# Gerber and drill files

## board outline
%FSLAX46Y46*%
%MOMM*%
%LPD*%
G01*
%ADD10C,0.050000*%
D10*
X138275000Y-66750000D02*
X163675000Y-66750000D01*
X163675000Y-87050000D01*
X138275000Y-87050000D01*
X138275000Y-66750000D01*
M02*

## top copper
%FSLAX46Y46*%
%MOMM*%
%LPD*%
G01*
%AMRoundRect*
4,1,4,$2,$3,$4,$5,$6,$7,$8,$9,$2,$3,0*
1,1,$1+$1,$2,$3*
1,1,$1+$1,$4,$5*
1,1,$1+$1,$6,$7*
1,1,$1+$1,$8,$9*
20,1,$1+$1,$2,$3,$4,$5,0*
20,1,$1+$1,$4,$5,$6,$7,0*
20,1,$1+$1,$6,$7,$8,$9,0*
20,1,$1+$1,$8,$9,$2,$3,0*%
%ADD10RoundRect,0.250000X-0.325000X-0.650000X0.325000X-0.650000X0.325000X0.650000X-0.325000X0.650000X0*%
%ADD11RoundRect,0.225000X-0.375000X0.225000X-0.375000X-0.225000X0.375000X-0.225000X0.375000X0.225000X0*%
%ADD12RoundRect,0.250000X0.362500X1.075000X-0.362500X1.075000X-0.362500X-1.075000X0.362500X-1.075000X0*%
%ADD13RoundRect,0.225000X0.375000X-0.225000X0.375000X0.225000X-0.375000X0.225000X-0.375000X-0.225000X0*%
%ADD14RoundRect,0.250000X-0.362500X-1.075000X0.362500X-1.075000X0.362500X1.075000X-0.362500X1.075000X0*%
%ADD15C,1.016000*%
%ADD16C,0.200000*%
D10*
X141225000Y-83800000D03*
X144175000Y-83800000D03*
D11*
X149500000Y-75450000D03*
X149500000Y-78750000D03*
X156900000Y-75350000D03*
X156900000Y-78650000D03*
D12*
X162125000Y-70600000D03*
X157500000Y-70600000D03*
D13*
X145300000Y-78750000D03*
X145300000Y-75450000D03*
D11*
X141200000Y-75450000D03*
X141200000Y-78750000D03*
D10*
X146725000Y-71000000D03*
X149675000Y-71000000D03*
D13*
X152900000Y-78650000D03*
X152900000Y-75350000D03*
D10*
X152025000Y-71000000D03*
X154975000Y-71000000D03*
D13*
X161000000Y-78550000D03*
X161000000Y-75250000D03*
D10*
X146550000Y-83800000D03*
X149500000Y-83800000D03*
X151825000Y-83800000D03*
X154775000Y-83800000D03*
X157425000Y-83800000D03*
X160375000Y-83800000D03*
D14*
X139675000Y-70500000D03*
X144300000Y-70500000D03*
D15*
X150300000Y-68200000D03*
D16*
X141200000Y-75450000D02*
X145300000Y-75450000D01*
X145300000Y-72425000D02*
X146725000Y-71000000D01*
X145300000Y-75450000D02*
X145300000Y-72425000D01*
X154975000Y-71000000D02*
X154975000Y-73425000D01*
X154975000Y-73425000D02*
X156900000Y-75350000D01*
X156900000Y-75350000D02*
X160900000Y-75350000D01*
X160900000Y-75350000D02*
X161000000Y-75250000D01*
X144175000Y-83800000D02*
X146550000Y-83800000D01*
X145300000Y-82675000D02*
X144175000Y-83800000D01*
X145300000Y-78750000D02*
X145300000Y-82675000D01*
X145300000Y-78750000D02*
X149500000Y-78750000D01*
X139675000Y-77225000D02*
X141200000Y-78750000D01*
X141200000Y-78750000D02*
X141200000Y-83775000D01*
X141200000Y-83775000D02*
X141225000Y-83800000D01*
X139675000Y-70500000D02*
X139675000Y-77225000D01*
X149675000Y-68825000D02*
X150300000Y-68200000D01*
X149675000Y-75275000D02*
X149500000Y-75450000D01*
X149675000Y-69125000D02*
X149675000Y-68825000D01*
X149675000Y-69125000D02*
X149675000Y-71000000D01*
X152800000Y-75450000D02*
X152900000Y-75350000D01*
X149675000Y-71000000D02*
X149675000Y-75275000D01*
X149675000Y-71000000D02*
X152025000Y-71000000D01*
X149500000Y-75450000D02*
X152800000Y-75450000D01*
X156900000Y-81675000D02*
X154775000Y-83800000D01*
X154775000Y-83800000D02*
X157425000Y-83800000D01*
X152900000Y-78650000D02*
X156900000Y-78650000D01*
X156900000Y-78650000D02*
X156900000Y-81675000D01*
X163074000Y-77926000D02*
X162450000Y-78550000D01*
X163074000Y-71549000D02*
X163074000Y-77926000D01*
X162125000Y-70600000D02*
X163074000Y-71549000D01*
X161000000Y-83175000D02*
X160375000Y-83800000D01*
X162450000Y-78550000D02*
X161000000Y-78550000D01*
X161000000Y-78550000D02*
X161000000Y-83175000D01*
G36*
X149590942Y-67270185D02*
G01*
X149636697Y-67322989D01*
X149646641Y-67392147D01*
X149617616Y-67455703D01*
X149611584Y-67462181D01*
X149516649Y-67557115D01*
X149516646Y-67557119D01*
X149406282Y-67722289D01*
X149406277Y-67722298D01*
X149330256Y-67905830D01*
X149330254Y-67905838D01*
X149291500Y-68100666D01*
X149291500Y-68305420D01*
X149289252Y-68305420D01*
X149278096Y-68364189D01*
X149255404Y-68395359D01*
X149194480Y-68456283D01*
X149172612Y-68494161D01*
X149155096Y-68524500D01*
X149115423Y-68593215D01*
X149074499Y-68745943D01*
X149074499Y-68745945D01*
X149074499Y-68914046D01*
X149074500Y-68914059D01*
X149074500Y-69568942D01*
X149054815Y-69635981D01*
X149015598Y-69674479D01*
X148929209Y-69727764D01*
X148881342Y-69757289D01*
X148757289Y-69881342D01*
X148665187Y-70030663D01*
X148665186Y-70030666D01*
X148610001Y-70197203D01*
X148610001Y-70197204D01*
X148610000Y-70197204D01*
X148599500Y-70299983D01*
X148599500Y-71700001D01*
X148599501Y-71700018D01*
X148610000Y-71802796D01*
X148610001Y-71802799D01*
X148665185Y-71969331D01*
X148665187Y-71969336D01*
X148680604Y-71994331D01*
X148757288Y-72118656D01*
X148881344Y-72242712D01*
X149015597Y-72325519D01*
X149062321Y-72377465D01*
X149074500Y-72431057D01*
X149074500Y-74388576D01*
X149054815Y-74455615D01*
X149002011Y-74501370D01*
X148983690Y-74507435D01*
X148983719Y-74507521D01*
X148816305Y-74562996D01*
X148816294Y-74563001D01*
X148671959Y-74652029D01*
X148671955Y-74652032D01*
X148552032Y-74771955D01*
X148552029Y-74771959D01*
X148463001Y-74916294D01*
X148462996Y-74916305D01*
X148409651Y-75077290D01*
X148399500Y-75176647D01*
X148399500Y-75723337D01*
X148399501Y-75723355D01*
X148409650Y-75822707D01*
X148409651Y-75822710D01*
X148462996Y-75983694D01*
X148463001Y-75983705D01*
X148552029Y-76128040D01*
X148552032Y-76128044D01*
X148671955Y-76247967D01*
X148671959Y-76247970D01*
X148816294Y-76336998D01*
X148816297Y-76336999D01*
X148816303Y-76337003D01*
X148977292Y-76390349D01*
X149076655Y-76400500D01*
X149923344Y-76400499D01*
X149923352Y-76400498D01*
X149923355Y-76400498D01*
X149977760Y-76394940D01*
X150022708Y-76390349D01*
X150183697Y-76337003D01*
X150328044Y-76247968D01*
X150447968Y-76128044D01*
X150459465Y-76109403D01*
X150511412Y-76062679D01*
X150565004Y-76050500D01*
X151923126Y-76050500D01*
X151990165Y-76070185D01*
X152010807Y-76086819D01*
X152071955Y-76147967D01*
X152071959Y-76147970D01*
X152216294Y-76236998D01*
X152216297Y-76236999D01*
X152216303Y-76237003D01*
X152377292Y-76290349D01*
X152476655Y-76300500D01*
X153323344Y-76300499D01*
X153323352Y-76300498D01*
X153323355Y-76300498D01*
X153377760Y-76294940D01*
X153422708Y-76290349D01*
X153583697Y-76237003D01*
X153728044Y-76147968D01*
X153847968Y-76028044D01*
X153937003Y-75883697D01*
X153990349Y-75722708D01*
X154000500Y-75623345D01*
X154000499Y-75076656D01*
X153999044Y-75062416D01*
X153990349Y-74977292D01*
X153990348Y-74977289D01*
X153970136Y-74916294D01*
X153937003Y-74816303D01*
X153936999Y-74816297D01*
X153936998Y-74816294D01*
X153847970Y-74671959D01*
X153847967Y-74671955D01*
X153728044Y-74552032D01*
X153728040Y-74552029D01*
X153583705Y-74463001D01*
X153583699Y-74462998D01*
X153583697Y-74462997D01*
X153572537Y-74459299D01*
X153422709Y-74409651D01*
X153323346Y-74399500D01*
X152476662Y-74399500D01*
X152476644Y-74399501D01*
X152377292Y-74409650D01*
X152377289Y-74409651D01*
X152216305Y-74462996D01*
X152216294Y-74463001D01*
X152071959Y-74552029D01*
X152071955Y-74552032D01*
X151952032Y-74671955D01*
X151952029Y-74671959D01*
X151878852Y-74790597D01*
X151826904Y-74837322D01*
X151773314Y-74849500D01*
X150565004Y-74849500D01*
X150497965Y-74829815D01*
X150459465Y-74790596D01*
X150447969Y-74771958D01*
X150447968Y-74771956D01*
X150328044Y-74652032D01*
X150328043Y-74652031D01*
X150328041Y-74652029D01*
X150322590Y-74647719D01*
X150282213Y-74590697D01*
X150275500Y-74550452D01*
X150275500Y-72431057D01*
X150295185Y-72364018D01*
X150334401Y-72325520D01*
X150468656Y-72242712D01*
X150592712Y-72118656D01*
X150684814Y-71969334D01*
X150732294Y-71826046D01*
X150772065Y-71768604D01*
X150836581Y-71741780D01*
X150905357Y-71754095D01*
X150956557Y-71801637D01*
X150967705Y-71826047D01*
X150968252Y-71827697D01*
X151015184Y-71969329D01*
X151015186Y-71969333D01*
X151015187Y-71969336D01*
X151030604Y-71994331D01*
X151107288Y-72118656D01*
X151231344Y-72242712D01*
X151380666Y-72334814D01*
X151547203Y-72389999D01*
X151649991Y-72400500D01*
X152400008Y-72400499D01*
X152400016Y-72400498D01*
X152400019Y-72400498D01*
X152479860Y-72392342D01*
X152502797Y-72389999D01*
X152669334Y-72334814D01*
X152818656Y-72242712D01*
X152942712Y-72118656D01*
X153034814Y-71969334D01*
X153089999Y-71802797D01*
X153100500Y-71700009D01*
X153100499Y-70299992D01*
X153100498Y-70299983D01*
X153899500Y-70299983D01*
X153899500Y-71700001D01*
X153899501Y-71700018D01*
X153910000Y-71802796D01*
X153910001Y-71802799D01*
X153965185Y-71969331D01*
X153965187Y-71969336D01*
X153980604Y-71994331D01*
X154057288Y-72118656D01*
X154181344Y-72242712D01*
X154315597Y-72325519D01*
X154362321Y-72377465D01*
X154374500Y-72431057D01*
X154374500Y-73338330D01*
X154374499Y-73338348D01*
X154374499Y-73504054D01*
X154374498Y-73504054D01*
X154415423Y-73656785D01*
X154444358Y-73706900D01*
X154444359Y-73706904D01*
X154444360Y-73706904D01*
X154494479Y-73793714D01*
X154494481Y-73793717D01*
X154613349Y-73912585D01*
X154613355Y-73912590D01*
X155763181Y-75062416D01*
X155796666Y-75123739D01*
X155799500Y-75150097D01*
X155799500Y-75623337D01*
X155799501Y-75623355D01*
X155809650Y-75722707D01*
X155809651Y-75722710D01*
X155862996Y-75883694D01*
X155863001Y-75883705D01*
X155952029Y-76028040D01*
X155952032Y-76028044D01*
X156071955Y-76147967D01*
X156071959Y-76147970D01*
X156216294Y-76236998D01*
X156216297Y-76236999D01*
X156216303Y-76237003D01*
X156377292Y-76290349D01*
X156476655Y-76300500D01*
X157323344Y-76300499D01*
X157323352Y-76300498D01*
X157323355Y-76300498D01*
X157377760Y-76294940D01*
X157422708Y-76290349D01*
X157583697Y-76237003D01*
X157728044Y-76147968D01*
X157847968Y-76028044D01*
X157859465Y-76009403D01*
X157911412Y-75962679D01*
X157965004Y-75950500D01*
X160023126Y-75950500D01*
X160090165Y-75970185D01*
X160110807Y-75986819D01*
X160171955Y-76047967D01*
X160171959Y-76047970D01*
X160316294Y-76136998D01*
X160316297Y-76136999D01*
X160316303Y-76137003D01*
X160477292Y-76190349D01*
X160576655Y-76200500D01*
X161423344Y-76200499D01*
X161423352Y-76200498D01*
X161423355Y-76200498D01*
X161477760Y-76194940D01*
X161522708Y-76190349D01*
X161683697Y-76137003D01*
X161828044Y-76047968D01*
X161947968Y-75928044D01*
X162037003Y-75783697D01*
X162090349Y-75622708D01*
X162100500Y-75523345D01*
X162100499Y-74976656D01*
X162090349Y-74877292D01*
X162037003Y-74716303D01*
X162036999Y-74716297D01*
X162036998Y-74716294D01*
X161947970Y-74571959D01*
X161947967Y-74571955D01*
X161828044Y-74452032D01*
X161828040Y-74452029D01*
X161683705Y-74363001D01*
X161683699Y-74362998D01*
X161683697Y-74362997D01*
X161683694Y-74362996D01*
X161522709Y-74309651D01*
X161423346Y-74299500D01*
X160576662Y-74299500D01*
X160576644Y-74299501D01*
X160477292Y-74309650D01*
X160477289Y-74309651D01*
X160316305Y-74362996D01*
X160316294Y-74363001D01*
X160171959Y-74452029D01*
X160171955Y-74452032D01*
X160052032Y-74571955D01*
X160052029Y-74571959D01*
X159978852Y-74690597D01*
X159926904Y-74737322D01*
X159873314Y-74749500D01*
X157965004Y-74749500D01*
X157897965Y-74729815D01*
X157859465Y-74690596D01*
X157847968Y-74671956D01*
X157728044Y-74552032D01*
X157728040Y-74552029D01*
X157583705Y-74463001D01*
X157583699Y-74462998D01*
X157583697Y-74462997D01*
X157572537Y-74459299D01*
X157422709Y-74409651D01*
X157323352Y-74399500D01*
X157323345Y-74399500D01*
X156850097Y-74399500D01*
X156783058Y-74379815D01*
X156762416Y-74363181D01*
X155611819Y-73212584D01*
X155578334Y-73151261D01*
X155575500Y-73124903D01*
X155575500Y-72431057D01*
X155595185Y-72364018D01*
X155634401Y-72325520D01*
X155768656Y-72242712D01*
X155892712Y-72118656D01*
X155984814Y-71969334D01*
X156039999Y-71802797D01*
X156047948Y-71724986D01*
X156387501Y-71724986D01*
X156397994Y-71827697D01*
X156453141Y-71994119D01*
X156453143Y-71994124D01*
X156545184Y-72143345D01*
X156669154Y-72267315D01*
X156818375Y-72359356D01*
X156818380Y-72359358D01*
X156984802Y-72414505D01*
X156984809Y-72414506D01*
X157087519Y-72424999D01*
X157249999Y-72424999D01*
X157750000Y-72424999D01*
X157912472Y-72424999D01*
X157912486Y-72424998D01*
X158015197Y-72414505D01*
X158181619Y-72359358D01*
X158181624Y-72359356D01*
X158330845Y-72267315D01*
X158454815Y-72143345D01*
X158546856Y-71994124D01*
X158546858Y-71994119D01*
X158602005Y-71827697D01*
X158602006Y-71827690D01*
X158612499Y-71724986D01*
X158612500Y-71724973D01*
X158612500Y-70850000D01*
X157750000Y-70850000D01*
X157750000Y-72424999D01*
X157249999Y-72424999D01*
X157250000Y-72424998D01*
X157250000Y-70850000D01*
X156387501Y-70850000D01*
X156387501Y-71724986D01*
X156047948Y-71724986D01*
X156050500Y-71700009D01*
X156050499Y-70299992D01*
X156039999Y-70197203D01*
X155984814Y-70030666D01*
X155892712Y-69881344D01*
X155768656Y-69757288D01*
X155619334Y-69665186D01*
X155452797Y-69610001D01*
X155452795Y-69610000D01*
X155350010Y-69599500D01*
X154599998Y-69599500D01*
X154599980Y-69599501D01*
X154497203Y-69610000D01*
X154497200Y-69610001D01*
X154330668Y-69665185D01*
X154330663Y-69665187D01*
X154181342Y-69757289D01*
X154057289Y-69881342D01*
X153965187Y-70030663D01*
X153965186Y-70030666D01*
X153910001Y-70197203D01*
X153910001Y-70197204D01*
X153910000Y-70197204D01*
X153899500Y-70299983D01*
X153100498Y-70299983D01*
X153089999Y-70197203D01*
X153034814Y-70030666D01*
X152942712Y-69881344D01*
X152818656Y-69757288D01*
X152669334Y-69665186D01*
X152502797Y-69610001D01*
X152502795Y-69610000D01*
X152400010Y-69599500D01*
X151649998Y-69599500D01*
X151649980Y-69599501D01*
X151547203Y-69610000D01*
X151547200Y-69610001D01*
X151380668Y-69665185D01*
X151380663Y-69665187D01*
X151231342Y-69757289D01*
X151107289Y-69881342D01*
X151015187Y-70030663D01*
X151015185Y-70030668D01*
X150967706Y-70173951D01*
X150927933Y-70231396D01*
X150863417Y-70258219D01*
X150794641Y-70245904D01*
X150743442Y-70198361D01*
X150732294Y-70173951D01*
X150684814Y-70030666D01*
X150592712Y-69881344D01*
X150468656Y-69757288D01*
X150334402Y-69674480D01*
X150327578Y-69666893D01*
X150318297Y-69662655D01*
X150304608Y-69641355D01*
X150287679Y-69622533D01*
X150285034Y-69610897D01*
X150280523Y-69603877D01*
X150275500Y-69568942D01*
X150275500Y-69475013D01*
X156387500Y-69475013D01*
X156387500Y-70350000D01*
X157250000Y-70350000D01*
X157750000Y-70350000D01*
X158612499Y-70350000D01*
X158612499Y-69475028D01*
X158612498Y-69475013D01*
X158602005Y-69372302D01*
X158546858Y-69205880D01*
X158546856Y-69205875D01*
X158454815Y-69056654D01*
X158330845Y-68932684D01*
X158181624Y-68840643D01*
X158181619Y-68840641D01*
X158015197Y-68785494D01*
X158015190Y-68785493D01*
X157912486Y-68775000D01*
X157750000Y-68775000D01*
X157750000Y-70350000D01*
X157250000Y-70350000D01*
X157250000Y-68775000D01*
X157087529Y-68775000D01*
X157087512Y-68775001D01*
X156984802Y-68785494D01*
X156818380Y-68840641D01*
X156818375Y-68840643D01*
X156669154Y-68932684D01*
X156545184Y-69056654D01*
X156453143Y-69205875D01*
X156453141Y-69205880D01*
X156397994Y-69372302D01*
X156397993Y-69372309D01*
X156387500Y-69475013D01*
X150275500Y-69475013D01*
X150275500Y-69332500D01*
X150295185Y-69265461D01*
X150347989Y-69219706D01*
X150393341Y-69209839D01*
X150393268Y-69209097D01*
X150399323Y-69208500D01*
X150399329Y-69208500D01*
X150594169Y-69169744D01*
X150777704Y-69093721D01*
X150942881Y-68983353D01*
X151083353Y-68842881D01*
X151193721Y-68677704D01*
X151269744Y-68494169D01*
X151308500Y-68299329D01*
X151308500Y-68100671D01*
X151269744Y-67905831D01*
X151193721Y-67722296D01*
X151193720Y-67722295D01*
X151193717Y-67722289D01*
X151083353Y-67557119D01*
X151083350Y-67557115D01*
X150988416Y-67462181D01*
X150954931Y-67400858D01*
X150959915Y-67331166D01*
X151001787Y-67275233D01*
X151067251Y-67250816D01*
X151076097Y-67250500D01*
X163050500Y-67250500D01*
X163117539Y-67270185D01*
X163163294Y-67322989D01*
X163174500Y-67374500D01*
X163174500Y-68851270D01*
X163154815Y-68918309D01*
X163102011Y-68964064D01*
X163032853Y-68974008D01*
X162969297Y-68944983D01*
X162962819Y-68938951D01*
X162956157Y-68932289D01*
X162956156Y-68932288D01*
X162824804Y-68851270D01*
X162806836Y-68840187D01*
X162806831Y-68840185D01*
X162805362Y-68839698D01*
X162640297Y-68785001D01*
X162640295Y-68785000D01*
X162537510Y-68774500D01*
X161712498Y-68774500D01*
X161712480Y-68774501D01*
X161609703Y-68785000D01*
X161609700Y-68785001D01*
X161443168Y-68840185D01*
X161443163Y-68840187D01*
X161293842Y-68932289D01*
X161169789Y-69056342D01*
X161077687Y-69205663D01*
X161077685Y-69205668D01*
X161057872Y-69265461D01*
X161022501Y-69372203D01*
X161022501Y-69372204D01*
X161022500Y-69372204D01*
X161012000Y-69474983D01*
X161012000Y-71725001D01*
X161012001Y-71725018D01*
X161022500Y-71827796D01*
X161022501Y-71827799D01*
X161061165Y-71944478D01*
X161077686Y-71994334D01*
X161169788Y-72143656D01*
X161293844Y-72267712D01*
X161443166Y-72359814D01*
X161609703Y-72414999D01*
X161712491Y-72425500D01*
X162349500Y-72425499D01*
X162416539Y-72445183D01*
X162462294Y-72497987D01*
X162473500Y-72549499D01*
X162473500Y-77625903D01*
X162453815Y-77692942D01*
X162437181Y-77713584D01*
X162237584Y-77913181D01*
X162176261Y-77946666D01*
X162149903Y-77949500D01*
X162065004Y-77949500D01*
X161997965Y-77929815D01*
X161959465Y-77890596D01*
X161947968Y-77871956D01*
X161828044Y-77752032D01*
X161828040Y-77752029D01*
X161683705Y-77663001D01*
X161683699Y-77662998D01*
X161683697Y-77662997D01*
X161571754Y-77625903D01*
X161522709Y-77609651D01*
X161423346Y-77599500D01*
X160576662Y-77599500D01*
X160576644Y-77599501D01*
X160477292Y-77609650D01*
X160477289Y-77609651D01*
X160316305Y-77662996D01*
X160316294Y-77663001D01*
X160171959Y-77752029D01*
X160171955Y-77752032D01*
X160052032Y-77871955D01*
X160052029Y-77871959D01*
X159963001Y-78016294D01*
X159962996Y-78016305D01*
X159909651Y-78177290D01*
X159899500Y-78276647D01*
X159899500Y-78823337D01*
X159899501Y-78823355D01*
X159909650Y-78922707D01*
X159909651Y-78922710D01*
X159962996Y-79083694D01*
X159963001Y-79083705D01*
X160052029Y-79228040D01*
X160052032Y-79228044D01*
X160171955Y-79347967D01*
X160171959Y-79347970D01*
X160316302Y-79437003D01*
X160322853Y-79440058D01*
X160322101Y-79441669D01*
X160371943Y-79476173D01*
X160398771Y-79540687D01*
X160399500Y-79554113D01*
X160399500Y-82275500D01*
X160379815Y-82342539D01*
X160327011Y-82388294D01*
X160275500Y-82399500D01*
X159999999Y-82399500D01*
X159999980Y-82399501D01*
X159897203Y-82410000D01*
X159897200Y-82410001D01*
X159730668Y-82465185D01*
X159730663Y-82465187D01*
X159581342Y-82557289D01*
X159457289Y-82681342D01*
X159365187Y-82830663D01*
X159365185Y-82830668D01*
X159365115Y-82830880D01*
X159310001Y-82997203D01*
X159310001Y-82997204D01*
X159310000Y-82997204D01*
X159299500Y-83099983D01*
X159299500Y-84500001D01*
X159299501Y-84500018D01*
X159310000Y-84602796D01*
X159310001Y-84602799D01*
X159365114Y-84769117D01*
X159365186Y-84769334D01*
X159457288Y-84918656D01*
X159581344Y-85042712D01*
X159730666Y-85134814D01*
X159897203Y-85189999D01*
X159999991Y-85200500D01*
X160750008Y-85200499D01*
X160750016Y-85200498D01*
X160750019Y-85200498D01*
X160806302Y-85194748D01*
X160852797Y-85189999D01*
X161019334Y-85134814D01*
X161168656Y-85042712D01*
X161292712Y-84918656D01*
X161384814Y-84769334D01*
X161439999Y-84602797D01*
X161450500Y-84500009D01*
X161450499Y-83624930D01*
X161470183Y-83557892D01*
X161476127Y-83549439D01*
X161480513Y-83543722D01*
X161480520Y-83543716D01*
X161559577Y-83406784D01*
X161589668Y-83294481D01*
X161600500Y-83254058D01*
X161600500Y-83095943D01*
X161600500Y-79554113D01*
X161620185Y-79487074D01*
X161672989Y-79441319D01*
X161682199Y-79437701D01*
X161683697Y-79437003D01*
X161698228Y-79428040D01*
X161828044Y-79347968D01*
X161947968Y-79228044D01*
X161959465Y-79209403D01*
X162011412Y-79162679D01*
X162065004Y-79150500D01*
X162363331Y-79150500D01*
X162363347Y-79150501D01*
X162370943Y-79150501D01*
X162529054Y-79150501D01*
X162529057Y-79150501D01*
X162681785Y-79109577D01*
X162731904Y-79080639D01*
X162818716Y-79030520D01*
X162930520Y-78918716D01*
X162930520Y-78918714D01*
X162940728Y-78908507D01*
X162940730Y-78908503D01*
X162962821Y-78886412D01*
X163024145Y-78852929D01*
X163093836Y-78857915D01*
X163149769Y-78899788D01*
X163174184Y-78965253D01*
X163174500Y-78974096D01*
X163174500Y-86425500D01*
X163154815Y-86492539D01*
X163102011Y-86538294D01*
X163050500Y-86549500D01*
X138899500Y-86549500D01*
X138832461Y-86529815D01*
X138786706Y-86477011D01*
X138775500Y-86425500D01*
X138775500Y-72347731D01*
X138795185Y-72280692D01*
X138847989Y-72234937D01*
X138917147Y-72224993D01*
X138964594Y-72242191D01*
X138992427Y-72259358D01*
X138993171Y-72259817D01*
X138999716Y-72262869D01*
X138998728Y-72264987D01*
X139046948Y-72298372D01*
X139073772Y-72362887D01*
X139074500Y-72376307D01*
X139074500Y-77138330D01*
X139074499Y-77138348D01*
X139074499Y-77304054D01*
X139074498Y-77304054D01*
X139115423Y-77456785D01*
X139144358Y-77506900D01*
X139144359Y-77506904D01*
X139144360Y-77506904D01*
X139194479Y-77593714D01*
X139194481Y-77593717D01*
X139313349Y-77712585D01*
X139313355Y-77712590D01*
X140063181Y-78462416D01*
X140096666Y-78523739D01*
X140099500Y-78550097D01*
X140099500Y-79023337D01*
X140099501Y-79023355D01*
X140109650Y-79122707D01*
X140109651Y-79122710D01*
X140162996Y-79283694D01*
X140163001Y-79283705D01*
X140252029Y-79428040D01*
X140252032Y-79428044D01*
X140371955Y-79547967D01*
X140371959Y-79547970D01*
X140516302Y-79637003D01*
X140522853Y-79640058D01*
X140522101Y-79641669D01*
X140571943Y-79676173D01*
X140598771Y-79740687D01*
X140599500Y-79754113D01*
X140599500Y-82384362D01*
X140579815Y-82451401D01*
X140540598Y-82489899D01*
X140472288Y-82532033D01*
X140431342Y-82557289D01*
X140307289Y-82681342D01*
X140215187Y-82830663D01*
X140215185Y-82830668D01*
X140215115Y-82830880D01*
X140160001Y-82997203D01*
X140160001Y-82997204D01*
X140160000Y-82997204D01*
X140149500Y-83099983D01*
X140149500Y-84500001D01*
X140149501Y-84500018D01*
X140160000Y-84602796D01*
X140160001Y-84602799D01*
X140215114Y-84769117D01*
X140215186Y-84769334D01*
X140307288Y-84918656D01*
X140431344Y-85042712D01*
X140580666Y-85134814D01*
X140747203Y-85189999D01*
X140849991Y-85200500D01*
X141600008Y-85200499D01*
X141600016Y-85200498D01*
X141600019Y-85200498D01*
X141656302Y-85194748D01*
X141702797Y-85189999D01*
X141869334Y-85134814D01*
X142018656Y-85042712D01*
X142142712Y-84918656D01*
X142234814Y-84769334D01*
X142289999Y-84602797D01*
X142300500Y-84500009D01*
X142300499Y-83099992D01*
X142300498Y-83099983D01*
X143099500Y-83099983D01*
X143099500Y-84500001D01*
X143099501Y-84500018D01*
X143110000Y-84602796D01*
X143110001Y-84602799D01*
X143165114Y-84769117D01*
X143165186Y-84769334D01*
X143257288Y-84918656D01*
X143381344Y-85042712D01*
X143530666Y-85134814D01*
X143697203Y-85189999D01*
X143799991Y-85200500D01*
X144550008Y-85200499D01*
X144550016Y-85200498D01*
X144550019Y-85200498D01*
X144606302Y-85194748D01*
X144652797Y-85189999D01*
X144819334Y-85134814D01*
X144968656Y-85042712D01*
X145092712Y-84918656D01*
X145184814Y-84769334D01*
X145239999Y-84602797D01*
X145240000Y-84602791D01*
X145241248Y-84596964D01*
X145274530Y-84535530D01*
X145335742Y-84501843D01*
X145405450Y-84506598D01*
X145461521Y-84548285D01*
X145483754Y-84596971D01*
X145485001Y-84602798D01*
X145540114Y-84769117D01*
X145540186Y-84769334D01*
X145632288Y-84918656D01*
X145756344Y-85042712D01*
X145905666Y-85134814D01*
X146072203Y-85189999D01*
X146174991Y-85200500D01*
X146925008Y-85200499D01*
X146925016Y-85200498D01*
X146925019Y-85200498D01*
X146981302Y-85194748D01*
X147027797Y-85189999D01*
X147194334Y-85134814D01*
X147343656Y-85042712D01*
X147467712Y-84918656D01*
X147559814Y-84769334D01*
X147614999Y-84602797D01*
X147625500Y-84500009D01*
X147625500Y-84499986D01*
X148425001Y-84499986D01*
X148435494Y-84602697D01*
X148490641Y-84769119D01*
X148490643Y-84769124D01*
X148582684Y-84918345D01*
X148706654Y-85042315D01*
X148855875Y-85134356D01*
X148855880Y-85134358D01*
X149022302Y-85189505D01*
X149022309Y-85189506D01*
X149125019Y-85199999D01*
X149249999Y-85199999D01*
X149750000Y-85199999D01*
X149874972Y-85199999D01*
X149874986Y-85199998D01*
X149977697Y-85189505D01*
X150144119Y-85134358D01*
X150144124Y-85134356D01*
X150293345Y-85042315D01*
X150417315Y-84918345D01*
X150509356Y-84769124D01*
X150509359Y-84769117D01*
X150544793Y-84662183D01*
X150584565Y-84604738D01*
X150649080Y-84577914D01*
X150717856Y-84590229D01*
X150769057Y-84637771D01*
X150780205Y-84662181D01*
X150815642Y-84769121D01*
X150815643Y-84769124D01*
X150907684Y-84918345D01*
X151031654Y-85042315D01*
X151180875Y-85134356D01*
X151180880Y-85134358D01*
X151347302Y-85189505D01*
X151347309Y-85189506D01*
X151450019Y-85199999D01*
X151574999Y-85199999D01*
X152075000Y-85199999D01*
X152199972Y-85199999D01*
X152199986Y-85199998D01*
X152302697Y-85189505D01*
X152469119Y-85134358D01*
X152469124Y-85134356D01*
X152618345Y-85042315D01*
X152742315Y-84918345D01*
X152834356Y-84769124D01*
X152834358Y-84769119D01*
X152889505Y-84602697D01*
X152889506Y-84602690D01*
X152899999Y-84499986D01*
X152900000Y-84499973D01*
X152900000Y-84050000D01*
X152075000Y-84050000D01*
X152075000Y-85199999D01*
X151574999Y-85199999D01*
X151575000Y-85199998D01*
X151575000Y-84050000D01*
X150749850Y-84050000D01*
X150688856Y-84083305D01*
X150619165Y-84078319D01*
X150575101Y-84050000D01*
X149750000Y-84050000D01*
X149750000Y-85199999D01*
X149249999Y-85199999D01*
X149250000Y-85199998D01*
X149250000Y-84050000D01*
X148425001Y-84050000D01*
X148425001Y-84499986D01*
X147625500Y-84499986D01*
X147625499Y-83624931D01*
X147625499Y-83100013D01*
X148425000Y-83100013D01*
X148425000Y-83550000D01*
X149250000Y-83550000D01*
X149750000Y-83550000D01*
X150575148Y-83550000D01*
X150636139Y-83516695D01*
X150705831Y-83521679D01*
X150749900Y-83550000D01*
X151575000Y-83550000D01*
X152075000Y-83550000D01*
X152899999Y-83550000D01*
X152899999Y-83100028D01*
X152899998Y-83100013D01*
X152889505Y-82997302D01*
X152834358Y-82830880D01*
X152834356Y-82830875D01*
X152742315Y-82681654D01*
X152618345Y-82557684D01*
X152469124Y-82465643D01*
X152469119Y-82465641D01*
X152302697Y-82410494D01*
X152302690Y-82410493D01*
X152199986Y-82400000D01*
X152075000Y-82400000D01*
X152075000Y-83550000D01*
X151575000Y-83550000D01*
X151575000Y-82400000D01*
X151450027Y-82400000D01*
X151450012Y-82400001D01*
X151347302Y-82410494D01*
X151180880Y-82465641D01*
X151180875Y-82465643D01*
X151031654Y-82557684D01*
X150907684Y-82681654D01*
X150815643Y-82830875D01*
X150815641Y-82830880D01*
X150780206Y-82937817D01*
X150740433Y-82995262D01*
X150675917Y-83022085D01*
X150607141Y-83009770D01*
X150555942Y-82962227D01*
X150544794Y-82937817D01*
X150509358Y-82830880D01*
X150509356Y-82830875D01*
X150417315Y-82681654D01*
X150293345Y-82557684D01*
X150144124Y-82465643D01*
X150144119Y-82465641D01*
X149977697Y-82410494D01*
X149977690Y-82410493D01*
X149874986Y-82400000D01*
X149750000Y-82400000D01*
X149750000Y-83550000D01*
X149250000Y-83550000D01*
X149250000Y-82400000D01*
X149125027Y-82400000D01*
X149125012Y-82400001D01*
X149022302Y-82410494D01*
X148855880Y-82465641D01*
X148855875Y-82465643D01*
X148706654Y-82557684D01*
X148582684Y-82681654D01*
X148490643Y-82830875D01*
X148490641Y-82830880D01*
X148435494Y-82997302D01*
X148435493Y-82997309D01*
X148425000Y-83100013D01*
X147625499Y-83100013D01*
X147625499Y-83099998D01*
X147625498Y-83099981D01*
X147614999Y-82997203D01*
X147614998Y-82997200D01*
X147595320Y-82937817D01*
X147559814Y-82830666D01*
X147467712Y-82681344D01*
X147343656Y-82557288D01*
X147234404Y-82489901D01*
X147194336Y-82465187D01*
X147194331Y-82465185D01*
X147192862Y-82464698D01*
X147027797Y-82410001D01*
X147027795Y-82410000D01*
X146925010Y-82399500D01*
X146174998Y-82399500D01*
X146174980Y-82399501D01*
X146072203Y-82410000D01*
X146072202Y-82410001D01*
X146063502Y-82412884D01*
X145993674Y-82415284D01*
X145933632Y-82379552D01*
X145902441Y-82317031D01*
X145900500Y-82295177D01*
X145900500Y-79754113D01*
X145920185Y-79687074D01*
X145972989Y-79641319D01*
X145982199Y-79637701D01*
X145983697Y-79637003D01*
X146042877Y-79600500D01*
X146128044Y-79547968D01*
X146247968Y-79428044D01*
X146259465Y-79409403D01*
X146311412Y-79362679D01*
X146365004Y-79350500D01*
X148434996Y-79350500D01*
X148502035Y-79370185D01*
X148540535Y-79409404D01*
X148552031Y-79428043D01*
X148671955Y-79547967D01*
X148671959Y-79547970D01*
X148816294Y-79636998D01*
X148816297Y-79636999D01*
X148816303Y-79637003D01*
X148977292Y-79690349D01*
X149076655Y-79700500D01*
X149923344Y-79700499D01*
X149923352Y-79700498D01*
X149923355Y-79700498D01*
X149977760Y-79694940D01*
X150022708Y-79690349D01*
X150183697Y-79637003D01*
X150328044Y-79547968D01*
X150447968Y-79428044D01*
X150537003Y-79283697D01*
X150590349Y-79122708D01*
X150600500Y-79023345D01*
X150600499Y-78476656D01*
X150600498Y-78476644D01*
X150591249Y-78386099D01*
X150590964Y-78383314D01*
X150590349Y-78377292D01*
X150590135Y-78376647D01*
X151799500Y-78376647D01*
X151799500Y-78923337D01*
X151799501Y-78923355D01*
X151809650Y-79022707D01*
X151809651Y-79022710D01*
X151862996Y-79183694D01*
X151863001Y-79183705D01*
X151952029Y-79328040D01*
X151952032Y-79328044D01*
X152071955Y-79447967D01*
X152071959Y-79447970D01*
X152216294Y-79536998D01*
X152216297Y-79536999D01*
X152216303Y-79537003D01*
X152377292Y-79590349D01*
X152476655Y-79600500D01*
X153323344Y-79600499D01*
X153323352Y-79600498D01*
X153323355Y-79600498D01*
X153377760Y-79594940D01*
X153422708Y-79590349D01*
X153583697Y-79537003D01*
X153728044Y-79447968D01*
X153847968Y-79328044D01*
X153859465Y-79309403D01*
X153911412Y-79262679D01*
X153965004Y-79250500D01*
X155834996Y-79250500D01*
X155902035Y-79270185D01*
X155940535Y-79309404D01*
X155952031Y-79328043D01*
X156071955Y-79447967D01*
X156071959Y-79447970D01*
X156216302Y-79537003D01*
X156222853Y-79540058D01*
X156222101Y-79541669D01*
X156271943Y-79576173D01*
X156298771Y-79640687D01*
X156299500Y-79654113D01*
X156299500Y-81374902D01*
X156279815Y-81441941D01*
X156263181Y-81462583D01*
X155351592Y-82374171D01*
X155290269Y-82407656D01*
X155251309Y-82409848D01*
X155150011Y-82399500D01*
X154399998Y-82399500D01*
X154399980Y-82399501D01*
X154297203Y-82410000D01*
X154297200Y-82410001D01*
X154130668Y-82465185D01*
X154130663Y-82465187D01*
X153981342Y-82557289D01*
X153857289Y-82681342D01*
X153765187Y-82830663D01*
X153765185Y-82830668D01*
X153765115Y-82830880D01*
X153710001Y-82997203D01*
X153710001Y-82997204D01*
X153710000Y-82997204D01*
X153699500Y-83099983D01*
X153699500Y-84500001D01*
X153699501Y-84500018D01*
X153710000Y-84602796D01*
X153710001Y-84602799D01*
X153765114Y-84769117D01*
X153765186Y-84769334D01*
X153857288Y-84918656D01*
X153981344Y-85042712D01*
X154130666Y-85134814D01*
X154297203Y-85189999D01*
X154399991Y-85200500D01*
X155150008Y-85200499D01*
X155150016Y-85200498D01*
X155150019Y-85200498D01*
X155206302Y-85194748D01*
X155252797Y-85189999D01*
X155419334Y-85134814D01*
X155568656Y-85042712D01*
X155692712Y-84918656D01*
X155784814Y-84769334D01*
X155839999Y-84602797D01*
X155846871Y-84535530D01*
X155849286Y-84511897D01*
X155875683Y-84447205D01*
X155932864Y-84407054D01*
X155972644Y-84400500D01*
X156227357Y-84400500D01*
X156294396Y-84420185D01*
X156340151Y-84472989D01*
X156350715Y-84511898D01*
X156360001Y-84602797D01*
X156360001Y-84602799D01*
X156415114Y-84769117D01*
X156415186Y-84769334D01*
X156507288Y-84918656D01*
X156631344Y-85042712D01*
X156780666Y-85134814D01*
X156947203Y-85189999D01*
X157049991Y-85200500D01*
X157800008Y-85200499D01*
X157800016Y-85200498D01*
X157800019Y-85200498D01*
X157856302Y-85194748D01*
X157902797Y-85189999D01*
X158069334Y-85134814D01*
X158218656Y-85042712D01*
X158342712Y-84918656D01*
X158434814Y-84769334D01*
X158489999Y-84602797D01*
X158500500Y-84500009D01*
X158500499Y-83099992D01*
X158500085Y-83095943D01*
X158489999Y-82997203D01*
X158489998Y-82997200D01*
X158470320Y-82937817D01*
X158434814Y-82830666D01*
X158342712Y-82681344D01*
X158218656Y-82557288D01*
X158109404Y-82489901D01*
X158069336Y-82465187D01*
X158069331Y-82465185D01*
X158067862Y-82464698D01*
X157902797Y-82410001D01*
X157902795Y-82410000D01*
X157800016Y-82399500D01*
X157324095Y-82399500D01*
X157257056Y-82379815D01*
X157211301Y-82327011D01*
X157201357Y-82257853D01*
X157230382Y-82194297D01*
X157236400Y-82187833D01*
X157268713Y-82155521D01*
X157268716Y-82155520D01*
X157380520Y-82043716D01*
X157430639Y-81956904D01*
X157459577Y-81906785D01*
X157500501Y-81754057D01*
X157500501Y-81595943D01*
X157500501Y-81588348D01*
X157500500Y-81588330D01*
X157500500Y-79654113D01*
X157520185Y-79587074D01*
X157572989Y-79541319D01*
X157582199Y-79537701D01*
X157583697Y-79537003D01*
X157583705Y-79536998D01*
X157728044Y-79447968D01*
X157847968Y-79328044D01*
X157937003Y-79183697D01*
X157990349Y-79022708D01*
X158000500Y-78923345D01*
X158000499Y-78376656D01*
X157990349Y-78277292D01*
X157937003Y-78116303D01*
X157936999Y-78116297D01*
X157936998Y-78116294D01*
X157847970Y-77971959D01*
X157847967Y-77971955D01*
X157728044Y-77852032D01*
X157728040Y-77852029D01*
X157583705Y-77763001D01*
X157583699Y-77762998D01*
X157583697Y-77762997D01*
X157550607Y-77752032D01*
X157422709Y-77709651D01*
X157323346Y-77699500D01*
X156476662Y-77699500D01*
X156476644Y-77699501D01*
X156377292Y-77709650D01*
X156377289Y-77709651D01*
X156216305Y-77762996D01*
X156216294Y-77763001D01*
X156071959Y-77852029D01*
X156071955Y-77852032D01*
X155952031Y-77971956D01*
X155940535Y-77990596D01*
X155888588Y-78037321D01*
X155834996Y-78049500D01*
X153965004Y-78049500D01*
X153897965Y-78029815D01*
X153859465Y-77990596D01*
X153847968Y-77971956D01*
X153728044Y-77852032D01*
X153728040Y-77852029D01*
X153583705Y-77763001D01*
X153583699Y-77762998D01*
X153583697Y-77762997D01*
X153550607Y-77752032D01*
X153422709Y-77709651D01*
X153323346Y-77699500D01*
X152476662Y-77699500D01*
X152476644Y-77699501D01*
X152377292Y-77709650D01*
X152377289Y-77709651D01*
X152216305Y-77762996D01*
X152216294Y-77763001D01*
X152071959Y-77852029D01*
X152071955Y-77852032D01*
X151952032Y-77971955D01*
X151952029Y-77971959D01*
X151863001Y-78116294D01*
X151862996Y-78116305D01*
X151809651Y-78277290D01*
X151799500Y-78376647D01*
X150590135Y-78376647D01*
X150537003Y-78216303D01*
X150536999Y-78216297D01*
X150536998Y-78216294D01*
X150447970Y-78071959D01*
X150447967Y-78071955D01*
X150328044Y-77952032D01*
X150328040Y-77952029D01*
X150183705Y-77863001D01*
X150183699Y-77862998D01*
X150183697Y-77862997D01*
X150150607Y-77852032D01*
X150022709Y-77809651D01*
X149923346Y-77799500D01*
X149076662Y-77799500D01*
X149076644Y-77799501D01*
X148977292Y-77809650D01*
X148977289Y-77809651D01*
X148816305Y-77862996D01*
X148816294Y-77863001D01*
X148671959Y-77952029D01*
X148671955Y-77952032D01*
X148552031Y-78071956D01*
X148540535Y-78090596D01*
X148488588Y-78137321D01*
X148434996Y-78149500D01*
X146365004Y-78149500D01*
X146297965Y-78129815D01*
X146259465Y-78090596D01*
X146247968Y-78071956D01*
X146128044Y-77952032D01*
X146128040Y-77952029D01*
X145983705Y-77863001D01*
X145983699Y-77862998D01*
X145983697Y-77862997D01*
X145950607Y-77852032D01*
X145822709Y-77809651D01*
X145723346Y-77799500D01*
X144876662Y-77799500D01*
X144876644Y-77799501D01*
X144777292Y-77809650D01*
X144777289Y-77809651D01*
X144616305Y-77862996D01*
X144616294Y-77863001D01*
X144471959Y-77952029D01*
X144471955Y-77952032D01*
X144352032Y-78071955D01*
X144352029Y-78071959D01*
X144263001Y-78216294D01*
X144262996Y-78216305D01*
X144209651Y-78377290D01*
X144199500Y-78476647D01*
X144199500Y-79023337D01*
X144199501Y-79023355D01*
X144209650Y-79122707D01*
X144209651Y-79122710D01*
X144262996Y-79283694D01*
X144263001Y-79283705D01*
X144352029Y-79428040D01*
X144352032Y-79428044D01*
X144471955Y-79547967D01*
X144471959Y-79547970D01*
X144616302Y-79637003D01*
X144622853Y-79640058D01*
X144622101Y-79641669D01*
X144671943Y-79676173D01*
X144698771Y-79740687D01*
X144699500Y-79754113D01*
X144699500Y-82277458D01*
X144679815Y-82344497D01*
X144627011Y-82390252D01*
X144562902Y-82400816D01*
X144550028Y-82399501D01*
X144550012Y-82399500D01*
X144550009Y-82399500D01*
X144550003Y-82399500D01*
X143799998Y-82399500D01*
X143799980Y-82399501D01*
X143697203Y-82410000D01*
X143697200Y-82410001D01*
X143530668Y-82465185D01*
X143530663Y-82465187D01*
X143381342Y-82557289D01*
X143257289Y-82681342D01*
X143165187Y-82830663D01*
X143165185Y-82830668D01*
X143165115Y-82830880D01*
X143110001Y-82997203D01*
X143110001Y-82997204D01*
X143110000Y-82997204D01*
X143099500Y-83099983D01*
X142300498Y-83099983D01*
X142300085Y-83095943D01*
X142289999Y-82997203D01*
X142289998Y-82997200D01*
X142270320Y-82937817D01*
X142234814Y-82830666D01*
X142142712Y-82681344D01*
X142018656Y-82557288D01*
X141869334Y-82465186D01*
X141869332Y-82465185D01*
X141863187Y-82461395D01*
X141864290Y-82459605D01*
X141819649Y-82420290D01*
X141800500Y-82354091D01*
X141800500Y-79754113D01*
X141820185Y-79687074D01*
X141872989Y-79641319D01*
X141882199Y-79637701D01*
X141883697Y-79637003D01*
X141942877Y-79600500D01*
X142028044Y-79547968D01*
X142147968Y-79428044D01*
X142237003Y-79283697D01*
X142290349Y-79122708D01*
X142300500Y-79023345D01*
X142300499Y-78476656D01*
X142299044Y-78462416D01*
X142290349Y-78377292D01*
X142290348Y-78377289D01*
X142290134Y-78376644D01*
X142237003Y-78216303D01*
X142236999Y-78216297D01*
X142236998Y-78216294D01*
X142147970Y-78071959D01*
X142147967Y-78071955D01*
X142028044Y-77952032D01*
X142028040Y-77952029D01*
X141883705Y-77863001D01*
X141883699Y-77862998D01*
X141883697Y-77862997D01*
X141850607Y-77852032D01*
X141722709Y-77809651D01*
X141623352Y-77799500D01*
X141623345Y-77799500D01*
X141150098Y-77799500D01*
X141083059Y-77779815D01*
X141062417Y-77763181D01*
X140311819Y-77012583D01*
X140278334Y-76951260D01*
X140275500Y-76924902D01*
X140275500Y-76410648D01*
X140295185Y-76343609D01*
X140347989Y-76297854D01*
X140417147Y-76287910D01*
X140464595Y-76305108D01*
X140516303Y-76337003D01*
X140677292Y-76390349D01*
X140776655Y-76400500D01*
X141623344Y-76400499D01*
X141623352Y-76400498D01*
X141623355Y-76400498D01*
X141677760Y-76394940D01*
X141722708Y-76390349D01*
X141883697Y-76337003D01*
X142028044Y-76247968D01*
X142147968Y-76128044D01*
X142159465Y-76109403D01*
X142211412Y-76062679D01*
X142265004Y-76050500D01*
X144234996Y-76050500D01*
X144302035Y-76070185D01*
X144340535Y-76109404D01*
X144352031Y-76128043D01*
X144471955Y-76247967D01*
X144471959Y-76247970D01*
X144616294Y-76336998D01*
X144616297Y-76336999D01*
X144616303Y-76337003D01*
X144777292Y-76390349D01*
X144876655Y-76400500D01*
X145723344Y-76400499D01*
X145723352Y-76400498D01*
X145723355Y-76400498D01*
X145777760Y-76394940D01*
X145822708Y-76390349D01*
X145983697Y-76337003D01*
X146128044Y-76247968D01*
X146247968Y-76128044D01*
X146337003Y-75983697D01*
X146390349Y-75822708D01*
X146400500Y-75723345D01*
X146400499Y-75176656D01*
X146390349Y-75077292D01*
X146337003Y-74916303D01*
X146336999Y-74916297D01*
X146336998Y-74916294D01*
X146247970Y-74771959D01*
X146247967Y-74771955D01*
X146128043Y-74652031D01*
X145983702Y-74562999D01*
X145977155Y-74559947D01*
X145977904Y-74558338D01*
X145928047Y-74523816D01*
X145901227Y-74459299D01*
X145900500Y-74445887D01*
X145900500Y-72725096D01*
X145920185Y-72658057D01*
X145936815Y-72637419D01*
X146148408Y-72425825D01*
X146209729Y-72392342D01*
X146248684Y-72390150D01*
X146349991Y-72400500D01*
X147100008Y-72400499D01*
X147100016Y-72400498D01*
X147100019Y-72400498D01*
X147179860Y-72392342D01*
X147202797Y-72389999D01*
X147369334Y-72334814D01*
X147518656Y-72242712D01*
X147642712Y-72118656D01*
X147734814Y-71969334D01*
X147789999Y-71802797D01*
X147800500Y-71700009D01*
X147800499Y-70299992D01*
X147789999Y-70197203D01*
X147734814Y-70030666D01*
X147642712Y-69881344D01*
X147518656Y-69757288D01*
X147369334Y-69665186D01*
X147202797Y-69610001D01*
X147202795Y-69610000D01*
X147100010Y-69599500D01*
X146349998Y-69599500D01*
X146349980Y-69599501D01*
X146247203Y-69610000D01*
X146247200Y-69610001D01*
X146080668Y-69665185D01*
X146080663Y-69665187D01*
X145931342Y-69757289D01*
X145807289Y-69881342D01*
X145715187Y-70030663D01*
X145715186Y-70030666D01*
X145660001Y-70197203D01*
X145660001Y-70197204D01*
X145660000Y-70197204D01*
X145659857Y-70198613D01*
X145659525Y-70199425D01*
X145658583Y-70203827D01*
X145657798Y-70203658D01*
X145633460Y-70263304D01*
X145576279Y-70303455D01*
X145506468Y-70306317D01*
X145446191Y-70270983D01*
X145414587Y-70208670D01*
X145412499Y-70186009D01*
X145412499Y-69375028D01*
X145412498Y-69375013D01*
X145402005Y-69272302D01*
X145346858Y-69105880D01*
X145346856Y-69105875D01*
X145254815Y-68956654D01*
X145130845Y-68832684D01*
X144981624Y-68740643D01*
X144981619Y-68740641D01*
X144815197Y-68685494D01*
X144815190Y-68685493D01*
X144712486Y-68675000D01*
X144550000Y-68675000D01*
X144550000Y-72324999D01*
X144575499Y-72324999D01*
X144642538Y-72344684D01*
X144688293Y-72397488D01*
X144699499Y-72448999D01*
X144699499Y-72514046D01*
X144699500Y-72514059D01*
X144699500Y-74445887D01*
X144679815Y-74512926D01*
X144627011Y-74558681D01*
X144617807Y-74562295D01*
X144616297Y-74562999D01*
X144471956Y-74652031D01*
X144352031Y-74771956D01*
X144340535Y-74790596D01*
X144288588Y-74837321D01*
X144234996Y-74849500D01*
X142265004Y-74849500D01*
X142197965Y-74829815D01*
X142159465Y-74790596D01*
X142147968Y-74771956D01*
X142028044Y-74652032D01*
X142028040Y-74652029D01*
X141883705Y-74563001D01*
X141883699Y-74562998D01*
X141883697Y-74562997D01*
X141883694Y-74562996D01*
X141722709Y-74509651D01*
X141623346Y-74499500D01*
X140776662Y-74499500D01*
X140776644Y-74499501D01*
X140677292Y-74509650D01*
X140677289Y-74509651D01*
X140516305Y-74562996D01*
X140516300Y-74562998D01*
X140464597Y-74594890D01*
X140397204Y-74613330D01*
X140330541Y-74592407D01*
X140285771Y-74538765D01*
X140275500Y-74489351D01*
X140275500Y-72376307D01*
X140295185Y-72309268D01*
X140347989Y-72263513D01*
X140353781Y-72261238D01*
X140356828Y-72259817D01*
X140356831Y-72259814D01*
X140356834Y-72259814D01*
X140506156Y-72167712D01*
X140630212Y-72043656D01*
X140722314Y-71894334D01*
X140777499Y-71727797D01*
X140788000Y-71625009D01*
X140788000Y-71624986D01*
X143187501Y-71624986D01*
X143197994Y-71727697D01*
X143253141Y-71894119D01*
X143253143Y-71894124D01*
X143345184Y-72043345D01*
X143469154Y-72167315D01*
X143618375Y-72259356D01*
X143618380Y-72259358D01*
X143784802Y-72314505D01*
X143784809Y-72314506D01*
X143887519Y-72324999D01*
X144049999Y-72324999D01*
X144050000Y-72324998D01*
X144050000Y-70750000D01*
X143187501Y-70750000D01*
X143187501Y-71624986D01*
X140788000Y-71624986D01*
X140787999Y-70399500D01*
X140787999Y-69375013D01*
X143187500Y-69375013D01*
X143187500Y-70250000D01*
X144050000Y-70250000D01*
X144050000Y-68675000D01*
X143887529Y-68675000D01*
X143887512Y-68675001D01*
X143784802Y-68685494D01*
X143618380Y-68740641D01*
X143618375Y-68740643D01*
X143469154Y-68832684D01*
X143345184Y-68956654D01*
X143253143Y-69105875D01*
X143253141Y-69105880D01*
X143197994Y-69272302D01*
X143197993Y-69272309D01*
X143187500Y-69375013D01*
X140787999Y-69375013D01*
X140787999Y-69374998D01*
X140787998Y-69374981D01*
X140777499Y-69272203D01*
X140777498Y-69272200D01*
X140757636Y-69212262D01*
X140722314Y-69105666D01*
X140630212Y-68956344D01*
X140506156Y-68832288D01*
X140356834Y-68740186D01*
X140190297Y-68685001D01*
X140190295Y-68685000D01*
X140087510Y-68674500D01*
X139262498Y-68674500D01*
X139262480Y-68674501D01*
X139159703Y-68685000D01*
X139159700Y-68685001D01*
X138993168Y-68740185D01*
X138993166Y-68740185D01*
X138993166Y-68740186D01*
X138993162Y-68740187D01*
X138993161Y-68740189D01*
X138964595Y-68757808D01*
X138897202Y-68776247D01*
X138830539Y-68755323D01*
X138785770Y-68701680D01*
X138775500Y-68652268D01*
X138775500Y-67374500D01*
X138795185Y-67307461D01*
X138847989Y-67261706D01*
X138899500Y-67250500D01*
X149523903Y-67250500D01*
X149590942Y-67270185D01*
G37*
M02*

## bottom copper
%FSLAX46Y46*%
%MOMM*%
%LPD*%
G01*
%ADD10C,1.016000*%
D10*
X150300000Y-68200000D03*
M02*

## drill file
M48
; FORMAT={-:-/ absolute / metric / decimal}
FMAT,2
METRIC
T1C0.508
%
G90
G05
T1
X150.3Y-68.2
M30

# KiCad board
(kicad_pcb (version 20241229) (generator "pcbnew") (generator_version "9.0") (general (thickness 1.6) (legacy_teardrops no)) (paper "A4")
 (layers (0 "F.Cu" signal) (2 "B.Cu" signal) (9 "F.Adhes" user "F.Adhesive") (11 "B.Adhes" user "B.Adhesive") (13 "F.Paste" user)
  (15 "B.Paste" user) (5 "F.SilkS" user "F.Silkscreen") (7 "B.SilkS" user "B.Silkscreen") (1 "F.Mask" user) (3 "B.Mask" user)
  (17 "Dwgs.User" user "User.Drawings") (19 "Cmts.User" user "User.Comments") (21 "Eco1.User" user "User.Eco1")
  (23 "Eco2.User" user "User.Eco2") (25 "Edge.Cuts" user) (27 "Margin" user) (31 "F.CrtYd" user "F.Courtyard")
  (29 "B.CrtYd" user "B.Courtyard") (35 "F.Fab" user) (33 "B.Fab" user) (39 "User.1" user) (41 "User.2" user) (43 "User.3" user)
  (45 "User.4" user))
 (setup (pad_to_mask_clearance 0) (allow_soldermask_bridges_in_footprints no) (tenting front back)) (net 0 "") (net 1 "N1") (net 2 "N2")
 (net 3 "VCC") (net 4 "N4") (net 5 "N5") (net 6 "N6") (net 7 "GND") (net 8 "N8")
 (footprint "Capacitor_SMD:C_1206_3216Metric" (layer "F.Cu") (at 142.7 83.8)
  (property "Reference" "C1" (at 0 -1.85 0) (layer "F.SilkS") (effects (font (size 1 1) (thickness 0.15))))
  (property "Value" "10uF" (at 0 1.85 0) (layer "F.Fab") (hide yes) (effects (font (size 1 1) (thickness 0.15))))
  (pad "1" smd roundrect (at -1.475 0) (size 1.15 1.8) (layers "F.Cu" "F.Mask" "F.Paste") (roundrect_rratio 0.217391) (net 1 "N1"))
  (pad "2" smd roundrect (at 1.475 0) (size 1.15 1.8) (layers "F.Cu" "F.Mask" "F.Paste") (roundrect_rratio 0.217391) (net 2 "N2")))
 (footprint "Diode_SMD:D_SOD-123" (layer "F.Cu") (at 149.5 77.1 -90)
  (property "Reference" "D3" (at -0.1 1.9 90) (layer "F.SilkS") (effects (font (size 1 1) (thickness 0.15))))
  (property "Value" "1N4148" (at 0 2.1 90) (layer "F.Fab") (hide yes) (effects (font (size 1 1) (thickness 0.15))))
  (pad "1" smd roundrect (at -1.65 0 270) (size 0.9 1.2) (layers "F.Cu" "F.Mask" "F.Paste") (roundrect_rratio 0.25) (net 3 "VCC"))
  (pad "2" smd roundrect (at 1.65 0 270) (size 0.9 1.2) (layers "F.Cu" "F.Mask" "F.Paste") (roundrect_rratio 0.25) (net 2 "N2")))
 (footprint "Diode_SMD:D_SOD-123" (layer "F.Cu") (at 156.9 77 -90)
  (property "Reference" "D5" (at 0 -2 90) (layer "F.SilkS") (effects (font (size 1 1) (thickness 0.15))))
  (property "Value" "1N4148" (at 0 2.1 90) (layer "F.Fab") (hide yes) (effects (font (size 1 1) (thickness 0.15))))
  (pad "1" smd roundrect (at -1.65 0 270) (size 0.9 1.2) (layers "F.Cu" "F.Mask" "F.Paste") (roundrect_rratio 0.25) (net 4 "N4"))
  (pad "2" smd roundrect (at 1.65 0 270) (size 0.9 1.2) (layers "F.Cu" "F.Mask" "F.Paste") (roundrect_rratio 0.25) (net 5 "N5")))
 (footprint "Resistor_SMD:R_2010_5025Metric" (layer "F.Cu") (at 159.8125 70.6 180)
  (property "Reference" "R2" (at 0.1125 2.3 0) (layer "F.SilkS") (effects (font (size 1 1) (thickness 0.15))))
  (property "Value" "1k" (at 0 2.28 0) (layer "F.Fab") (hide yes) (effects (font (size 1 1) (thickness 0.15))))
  (pad "1" smd roundrect (at -2.3125 0 180) (size 1.225 2.65) (layers "F.Cu" "F.Mask" "F.Paste") (roundrect_rratio 0.204082) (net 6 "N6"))
  (pad "2" smd roundrect (at 2.3125 0 180) (size 1.225 2.65) (layers "F.Cu" "F.Mask" "F.Paste") (roundrect_rratio 0.204082) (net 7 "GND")))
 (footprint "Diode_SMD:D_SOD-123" (layer "F.Cu") (at 145.3 77.1 90)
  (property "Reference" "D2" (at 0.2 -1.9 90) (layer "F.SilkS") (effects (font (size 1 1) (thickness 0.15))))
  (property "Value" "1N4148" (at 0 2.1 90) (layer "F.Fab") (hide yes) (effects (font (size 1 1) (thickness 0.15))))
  (pad "1" smd roundrect (at -1.65 0 90) (size 0.9 1.2) (layers "F.Cu" "F.Mask" "F.Paste") (roundrect_rratio 0.25) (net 2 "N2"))
  (pad "2" smd roundrect (at 1.65 0 90) (size 0.9 1.2) (layers "F.Cu" "F.Mask" "F.Paste") (roundrect_rratio 0.25) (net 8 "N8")))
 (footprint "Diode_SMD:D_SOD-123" (layer "F.Cu") (at 141.2 77.1 -90)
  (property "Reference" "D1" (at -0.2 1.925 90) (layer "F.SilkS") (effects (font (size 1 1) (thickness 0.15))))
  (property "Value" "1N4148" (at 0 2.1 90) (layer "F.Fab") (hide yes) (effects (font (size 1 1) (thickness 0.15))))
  (pad "1" smd roundrect (at -1.65 0 270) (size 0.9 1.2) (layers "F.Cu" "F.Mask" "F.Paste") (roundrect_rratio 0.25) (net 8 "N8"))
  (pad "2" smd roundrect (at 1.65 0 270) (size 0.9 1.2) (layers "F.Cu" "F.Mask" "F.Paste") (roundrect_rratio 0.25) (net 1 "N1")))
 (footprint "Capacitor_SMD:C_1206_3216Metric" (layer "F.Cu") (at 148.2 71)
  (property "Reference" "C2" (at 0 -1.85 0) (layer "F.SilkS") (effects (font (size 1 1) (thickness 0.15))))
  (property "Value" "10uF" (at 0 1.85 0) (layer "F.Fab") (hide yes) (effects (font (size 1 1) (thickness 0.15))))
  (pad "1" smd roundrect (at -1.475 0) (size 1.15 1.8) (layers "F.Cu" "F.Mask" "F.Paste") (roundrect_rratio 0.217391) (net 8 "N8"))
  (pad "2" smd roundrect (at 1.475 0) (size 1.15 1.8) (layers "F.Cu" "F.Mask" "F.Paste") (roundrect_rratio 0.217391) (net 3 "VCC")))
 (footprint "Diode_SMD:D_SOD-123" (layer "F.Cu") (at 152.9 77 90)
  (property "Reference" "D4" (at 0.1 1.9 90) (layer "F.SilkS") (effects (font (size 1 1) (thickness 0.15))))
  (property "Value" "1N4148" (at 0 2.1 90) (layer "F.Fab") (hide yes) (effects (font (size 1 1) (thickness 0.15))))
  (pad "1" smd roundrect (at -1.65 0 90) (size 0.9 1.2) (layers "F.Cu" "F.Mask" "F.Paste") (roundrect_rratio 0.25) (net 5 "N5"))
  (pad "2" smd roundrect (at 1.65 0 90) (size 0.9 1.2) (layers "F.Cu" "F.Mask" "F.Paste") (roundrect_rratio 0.25) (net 3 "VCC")))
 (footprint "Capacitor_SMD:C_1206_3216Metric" (layer "F.Cu") (at 153.5 71)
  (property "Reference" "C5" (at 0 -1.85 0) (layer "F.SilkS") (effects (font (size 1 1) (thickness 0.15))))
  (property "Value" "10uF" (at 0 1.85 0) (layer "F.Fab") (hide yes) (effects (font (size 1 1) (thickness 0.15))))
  (pad "1" smd roundrect (at -1.475 0) (size 1.15 1.8) (layers "F.Cu" "F.Mask" "F.Paste") (roundrect_rratio 0.217391) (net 3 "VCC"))
  (pad "2" smd roundrect (at 1.475 0) (size 1.15 1.8) (layers "F.Cu" "F.Mask" "F.Paste") (roundrect_rratio 0.217391) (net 4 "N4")))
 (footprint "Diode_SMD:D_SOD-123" (layer "F.Cu") (at 161 76.9 90)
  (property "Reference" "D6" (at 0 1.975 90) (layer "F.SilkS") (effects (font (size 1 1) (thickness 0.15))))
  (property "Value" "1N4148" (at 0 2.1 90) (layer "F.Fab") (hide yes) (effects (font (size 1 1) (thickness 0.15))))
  (pad "1" smd roundrect (at -1.65 0 90) (size 0.9 1.2) (layers "F.Cu" "F.Mask" "F.Paste") (roundrect_rratio 0.25) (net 6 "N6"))
  (pad "2" smd roundrect (at 1.65 0 90) (size 0.9 1.2) (layers "F.Cu" "F.Mask" "F.Paste") (roundrect_rratio 0.25) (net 4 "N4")))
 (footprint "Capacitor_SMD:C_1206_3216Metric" (layer "F.Cu") (at 148.025 83.8)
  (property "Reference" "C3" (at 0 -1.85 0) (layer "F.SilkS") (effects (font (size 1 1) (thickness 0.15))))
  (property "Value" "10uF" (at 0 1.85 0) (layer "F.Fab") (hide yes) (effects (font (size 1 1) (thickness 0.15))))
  (pad "1" smd roundrect (at -1.475 0) (size 1.15 1.8) (layers "F.Cu" "F.Mask" "F.Paste") (roundrect_rratio 0.217391) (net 2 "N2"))
  (pad "2" smd roundrect (at 1.475 0) (size 1.15 1.8) (layers "F.Cu" "F.Mask" "F.Paste") (roundrect_rratio 0.217391) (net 7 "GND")))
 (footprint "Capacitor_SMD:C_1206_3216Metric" (layer "F.Cu") (at 153.3 83.8)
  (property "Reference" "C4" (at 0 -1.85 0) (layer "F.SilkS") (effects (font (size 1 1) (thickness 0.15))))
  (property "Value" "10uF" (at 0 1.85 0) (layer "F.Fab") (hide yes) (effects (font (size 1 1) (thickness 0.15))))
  (pad "1" smd roundrect (at -1.475 0) (size 1.15 1.8) (layers "F.Cu" "F.Mask" "F.Paste") (roundrect_rratio 0.217391) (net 7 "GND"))
  (pad "2" smd roundrect (at 1.475 0) (size 1.15 1.8) (layers "F.Cu" "F.Mask" "F.Paste") (roundrect_rratio 0.217391) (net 5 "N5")))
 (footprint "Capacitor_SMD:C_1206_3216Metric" (layer "F.Cu") (at 158.9 83.8)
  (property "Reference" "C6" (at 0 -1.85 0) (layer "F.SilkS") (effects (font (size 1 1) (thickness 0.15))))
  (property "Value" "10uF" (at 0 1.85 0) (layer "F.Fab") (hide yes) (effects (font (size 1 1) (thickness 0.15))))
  (pad "1" smd roundrect (at -1.475 0) (size 1.15 1.8) (layers "F.Cu" "F.Mask" "F.Paste") (roundrect_rratio 0.217391) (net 5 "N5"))
  (pad "2" smd roundrect (at 1.475 0) (size 1.15 1.8) (layers "F.Cu" "F.Mask" "F.Paste") (roundrect_rratio 0.217391) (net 6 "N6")))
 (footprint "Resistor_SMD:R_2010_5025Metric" (layer "F.Cu") (at 141.9875 70.5)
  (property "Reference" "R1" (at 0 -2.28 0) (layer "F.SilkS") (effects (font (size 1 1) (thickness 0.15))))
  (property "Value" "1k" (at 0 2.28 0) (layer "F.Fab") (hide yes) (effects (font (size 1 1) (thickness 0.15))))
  (pad "1" smd roundrect (at -2.3125 0) (size 1.225 2.65) (layers "F.Cu" "F.Mask" "F.Paste") (roundrect_rratio 0.204082) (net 1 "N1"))
  (pad "2" smd roundrect (at 2.3125 0) (size 1.225 2.65) (layers "F.Cu" "F.Mask" "F.Paste") (roundrect_rratio 0.204082) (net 7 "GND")))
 (gr_rect (start 138.275 66.75) (end 163.675 87.05) (stroke (width 0.05) (type default)) (fill no) (layer "Edge.Cuts"))
 (segment (start 141.2 75.45) (end 145.3 75.45) (width 0.2) (layer "F.Cu") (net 8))
 (segment (start 145.3 72.425) (end 146.725 71) (width 0.2) (layer "F.Cu") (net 8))
 (segment (start 145.3 75.45) (end 145.3 72.425) (width 0.2) (layer "F.Cu") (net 8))
 (segment (start 154.975 71) (end 154.975 73.425) (width 0.2) (layer "F.Cu") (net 4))
 (segment (start 154.975 73.425) (end 156.9 75.35) (width 0.2) (layer "F.Cu") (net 4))
 (segment (start 156.9 75.35) (end 160.9 75.35) (width 0.2) (layer "F.Cu") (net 4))
 (segment (start 160.9 75.35) (end 161 75.25) (width 0.2) (layer "F.Cu") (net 4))
 (segment (start 144.175 83.8) (end 146.55 83.8) (width 0.2) (layer "F.Cu") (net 2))
 (segment (start 145.3 82.675) (end 144.175 83.8) (width 0.2) (layer "F.Cu") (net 2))
 (segment (start 145.3 78.75) (end 145.3 82.675) (width 0.2) (layer "F.Cu") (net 2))
 (segment (start 145.3 78.75) (end 149.5 78.75) (width 0.2) (layer "F.Cu") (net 2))
 (segment (start 139.675 77.225) (end 141.2 78.75) (width 0.2) (layer "F.Cu") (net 1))
 (segment (start 141.2 78.75) (end 141.2 83.775) (width 0.2) (layer "F.Cu") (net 1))
 (segment (start 141.2 83.775) (end 141.225 83.8) (width 0.2) (layer "F.Cu") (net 1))
 (segment (start 139.675 70.5) (end 139.675 77.225) (width 0.2) (layer "F.Cu") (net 1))
 (segment (start 149.675 68.825) (end 150.3 68.2) (width 0.2) (layer "F.Cu") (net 3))
 (segment (start 149.675 75.275) (end 149.5 75.45) (width 0.2) (layer "F.Cu") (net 3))
 (segment (start 149.675 69.125) (end 149.675 68.825) (width 0.2) (layer "F.Cu") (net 3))
 (segment (start 149.675 69.125) (end 149.675 71) (width 0.2) (layer "F.Cu") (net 3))
 (segment (start 152.8 75.45) (end 152.9 75.35) (width 0.2) (layer "F.Cu") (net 3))
 (segment (start 149.675 71) (end 149.675 75.275) (width 0.2) (layer "F.Cu") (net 3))
 (segment (start 149.675 71) (end 152.025 71) (width 0.2) (layer "F.Cu") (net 3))
 (segment (start 149.5 75.45) (end 152.8 75.45) (width 0.2) (layer "F.Cu") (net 3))
 (via (at 150.3 68.2) (size 1.016) (drill 0.508) (layers "F.Cu" "B.Cu") (tenting none) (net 3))
 (segment (start 156.9 81.675) (end 154.775 83.8) (width 0.2) (layer "F.Cu") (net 5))
 (segment (start 154.775 83.8) (end 157.425 83.8) (width 0.2) (layer "F.Cu") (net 5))
 (segment (start 152.9 78.65) (end 156.9 78.65) (width 0.2) (layer "F.Cu") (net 5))
 (segment (start 156.9 78.65) (end 156.9 81.675) (width 0.2) (layer "F.Cu") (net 5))
 (segment (start 163.074 77.926) (end 162.45 78.55) (width 0.2) (layer "F.Cu") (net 6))
 (segment (start 163.074 71.549) (end 163.074 77.926) (width 0.2) (layer "F.Cu") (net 6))
 (segment (start 162.125 70.6) (end 163.074 71.549) (width 0.2) (layer "F.Cu") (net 6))
 (segment (start 161 83.175) (end 160.375 83.8) (width 0.2) (layer "F.Cu") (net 6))
 (segment (start 162.45 78.55) (end 161 78.55) (width 0.2) (layer "F.Cu") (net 6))
 (segment (start 161 78.55) (end 161 83.175) (width 0.2) (layer "F.Cu") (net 6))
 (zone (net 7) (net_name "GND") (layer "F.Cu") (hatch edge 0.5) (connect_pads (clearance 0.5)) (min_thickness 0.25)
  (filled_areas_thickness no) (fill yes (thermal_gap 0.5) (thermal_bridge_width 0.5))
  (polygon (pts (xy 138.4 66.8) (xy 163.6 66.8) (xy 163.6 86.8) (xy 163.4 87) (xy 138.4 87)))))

